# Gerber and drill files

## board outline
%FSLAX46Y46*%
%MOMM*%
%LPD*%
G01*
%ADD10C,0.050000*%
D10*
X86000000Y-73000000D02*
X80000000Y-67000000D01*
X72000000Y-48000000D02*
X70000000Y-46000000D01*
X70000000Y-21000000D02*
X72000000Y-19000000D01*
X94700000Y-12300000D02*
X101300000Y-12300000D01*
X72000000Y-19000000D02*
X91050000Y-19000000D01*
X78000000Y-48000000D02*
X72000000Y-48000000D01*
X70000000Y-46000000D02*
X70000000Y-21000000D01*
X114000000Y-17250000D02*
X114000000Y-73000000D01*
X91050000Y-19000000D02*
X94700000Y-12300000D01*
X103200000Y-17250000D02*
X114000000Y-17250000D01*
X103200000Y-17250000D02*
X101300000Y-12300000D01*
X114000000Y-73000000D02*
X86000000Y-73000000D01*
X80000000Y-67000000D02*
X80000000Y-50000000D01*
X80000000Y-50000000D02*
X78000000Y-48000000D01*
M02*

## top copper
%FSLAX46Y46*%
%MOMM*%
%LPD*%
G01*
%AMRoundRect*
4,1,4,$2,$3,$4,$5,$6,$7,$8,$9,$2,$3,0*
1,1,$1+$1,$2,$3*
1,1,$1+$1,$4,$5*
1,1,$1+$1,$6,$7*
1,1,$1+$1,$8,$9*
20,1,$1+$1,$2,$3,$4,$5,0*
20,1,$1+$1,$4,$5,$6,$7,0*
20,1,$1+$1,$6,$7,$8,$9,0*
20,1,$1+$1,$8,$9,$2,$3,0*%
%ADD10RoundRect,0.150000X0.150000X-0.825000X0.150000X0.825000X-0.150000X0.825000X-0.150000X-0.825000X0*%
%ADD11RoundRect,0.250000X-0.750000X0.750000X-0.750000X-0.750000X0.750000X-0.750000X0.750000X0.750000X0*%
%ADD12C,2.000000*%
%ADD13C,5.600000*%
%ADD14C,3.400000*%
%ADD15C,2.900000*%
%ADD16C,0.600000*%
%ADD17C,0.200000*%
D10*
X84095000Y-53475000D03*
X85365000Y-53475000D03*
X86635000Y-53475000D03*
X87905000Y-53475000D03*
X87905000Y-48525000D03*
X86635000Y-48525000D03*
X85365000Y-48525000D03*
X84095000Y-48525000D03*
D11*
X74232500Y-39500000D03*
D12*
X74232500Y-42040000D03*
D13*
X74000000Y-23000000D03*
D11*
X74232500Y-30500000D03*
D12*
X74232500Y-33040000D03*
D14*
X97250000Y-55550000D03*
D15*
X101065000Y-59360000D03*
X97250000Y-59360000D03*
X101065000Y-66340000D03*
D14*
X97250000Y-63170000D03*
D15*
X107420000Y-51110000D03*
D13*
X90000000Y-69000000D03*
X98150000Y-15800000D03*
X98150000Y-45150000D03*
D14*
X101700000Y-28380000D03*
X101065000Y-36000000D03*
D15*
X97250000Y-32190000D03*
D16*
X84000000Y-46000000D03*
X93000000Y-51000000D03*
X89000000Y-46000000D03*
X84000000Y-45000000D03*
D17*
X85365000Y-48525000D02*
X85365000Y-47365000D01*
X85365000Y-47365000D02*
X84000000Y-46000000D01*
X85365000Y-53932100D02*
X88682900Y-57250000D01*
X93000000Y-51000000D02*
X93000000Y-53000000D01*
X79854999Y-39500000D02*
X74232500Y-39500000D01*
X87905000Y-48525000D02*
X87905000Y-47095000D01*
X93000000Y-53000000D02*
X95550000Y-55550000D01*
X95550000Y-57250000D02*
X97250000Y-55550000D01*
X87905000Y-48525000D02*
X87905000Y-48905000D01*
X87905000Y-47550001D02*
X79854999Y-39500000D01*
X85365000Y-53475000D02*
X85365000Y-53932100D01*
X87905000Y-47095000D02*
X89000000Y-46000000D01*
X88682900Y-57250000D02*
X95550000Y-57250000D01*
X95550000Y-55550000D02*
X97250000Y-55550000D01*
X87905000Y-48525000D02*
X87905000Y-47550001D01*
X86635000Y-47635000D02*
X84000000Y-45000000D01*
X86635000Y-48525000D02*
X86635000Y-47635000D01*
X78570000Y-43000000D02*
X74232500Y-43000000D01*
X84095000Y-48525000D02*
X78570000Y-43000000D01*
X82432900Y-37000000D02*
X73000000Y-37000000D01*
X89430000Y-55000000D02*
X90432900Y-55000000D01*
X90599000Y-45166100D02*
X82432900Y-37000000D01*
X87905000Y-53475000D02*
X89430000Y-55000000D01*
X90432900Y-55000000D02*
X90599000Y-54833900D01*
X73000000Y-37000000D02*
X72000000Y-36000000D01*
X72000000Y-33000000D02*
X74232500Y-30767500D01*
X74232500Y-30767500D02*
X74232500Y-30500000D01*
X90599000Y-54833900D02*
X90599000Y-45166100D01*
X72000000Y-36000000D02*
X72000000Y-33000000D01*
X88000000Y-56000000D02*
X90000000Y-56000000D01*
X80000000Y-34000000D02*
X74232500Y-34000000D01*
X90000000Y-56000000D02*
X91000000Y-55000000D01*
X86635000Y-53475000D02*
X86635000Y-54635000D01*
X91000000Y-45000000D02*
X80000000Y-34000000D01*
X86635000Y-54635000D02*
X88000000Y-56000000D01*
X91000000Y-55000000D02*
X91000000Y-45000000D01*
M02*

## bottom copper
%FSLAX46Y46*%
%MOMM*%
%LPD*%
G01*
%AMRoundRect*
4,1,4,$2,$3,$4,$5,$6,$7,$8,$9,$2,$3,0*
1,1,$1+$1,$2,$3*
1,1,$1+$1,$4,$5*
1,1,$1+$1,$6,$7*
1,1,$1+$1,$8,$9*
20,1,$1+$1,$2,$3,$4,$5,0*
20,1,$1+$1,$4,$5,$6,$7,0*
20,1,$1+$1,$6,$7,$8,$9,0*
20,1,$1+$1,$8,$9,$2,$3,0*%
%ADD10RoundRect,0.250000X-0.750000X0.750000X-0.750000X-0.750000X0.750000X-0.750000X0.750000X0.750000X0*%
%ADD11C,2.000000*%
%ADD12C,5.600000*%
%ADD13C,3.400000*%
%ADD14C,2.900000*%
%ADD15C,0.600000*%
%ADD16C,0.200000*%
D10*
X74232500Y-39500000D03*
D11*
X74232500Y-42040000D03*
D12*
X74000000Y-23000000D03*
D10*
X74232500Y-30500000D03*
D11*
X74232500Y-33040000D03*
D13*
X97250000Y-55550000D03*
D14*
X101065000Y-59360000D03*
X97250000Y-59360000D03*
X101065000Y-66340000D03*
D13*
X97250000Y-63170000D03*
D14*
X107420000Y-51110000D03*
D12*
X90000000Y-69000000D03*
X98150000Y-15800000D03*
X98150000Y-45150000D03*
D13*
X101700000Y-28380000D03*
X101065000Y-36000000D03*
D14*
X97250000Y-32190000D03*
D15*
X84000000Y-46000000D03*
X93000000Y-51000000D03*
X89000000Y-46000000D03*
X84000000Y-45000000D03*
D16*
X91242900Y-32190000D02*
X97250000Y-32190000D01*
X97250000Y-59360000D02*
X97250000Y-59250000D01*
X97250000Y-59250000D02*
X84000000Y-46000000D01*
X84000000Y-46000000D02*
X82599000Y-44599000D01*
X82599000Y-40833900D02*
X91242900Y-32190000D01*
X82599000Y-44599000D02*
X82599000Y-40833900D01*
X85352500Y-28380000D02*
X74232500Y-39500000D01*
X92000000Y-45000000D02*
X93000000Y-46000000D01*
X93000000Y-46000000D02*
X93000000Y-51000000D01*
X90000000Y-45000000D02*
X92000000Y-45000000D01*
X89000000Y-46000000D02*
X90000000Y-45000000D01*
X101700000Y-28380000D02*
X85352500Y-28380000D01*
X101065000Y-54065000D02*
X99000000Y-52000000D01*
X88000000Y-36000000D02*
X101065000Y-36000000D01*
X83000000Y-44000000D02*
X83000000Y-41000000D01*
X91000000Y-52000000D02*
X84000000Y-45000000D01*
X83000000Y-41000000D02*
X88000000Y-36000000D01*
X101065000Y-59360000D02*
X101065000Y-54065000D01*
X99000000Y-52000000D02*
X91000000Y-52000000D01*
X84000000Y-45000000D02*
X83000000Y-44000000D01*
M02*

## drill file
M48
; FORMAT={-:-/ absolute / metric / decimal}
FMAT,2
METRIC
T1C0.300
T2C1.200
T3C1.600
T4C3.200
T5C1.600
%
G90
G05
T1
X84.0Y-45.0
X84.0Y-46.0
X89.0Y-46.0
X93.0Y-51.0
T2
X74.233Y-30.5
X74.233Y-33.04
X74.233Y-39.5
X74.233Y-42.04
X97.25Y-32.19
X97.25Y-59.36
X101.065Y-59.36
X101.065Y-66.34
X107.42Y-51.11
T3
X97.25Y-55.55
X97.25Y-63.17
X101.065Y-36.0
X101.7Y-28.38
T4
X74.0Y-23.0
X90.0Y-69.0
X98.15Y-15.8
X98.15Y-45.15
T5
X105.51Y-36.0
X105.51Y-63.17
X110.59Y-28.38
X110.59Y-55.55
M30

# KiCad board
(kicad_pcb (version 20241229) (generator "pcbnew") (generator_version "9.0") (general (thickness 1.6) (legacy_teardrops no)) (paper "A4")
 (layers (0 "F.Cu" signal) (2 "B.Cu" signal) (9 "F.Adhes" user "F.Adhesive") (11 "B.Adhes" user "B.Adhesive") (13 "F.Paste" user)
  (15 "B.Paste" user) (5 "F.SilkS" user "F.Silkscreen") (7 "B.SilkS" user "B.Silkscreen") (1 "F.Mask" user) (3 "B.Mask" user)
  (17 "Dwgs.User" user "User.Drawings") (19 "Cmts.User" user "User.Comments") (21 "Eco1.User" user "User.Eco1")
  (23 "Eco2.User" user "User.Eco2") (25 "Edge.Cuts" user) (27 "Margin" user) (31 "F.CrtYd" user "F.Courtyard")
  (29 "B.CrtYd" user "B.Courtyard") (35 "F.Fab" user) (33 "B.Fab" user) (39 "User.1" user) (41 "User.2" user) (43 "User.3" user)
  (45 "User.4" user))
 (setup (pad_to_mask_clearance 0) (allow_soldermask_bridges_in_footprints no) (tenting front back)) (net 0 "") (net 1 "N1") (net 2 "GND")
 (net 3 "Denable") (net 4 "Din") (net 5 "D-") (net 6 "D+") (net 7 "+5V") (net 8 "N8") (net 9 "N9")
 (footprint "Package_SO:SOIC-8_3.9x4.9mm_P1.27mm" (layer "F.Cu") (at 86 51 90)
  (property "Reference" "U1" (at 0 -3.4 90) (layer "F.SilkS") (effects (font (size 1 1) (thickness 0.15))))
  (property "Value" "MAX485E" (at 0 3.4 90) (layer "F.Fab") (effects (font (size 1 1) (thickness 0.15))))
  (pad "1" smd roundrect (at -2.475 -1.905 90) (size 1.95 0.6) (layers "F.Cu" "F.Mask" "F.Paste") (roundrect_rratio 0.25) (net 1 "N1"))
  (pad "2" smd roundrect (at -2.475 -0.635 90) (size 1.95 0.6) (layers "F.Cu" "F.Mask" "F.Paste") (roundrect_rratio 0.25) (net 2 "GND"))
  (pad "3" smd roundrect (at -2.475 0.635 90) (size 1.95 0.6) (layers "F.Cu" "F.Mask" "F.Paste") (roundrect_rratio 0.25) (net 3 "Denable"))
  (pad "4" smd roundrect (at -2.475 1.905 90) (size 1.95 0.6) (layers "F.Cu" "F.Mask" "F.Paste") (roundrect_rratio 0.25) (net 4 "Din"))
  (pad "5" smd roundrect (at 2.475 1.905 90) (size 1.95 0.6) (layers "F.Cu" "F.Mask" "F.Paste") (roundrect_rratio 0.25) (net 2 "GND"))
  (pad "6" smd roundrect (at 2.475 0.635 90) (size 1.95 0.6) (layers "F.Cu" "F.Mask" "F.Paste") (roundrect_rratio 0.25) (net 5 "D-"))
  (pad "7" smd roundrect (at 2.475 -0.635 90) (size 1.95 0.6) (layers "F.Cu" "F.Mask" "F.Paste") (roundrect_rratio 0.25) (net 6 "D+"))
  (pad "8" smd roundrect (at 2.475 -1.905 90) (size 1.95 0.6) (layers "F.Cu" "F.Mask" "F.Paste") (roundrect_rratio 0.25) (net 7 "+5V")))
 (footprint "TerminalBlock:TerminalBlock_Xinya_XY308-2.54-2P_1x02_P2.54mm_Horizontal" (layer "F.Cu") (at 74.2325 39.5 -90)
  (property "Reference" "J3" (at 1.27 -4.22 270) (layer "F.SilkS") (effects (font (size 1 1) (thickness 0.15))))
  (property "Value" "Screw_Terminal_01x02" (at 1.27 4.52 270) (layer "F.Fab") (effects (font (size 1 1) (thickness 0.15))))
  (pad "1" thru_hole roundrect (at 0 0 270) (size 2 2) (drill 1.2) (layers "*.Cu" "*.Mask") (remove_unused_layers no)
   (roundrect_rratio 0.125) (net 2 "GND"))
  (pad "2" thru_hole circle (at 2.54 0 270) (size 2 2) (drill 1.2) (layers "*.Cu" "*.Mask") (remove_unused_layers no) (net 7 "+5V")))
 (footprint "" (layer "F.Cu") (at 74 23)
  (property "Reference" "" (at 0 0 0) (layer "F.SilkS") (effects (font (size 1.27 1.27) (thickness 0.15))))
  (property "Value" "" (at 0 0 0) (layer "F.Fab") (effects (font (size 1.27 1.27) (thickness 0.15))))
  (pad "1" thru_hole circle (at 0 0) (size 5.6 5.6) (drill 3.2) (layers "*.Cu" "*.Mask") (remove_unused_layers no) (zone_connect 2)))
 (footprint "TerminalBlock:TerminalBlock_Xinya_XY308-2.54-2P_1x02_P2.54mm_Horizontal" (layer "F.Cu") (at 74.2325 30.5 -90)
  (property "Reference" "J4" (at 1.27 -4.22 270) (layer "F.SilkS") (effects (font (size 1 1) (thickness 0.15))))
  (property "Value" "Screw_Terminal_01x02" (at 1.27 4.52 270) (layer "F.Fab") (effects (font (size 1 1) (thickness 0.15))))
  (pad "1" thru_hole roundrect (at 0 0 270) (size 2 2) (drill 1.2) (layers "*.Cu" "*.Mask") (remove_unused_layers no)
   (roundrect_rratio 0.125) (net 4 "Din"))
  (pad "2" thru_hole circle (at 2.54 0 270) (size 2 2) (drill 1.2) (layers "*.Cu" "*.Mask") (remove_unused_layers no) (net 3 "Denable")))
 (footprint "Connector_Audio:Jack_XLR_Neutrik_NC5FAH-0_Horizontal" (layer "F.Cu") (at 97.25 55.55)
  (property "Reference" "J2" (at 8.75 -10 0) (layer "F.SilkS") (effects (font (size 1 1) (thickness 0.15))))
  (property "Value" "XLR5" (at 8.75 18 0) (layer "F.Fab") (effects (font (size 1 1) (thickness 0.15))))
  (pad "" np_thru_hole circle (at 8.26 7.62) (size 1.6 1.6) (drill 1.6) (layers "*.Cu" "*.Mask"))
  (pad "" np_thru_hole circle (at 13.34 0) (size 1.6 1.6) (drill 1.6) (layers "*.Cu" "*.Mask"))
  (pad "1" thru_hole circle (at 0 0) (size 3.4 3.4) (drill 1.6) (layers "*.Cu" "*.Mask") (remove_unused_layers no) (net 2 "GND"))
  (pad "2" thru_hole circle (at 3.815 3.81) (size 2.9 2.9) (drill 1.2) (layers "*.Cu" "*.Mask") (remove_unused_layers no) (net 5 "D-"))
  (pad "3" thru_hole circle (at 0 3.81) (size 2.9 2.9) (drill 1.2) (layers "*.Cu" "*.Mask") (remove_unused_layers no) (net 6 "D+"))
  (pad "4" thru_hole circle (at 3.815 10.79) (size 2.9 2.9) (drill 1.2) (layers "*.Cu" "*.Mask") (remove_unused_layers no) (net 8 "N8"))
  (pad "5" thru_hole circle (at 0 7.62) (size 3.4 3.4) (drill 1.6) (layers "*.Cu" "*.Mask") (remove_unused_layers no) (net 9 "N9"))
  (pad "G" thru_hole circle (at 10.17 -4.44) (size 2.9 2.9) (drill 1.2) (layers "*.Cu" "*.Mask") (remove_unused_layers no)))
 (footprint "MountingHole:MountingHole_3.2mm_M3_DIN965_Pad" (layer "F.Cu") (at 90 69)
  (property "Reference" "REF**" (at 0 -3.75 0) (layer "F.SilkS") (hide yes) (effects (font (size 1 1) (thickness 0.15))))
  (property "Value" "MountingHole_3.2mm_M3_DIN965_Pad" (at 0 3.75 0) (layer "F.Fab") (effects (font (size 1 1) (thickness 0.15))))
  (pad "1" thru_hole circle (at 0 0) (size 5.6 5.6) (drill 3.2) (layers "*.Cu" "*.Mask") (remove_unused_layers no) (zone_connect 2)))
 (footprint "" (layer "F.Cu") (at 98.15 15.8)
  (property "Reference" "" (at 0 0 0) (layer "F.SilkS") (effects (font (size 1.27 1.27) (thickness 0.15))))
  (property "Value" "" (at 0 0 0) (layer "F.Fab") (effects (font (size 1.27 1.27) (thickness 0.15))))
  (pad "1" thru_hole circle (at 0 0) (size 5.6 5.6) (drill 3.2) (layers "*.Cu" "*.Mask") (remove_unused_layers no) (zone_connect 2)))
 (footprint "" (layer "F.Cu") (at 98.15 45.15)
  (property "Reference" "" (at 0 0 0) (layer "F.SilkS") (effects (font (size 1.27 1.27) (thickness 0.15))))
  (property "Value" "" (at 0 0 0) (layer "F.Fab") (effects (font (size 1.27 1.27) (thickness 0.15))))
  (pad "1" thru_hole circle (at 0 0) (size 5.6 5.6) (drill 3.2) (layers "*.Cu" "*.Mask") (remove_unused_layers no) (zone_connect 2)))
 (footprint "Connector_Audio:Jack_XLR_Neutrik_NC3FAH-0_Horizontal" (layer "F.Cu") (at 101.7 28.38)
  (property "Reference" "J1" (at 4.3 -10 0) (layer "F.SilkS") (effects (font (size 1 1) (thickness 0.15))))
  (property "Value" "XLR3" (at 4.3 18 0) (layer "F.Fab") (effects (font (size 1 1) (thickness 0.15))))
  (pad "" np_thru_hole circle (at 3.81 7.62) (size 1.6 1.6) (drill 1.6) (layers "*.Cu" "*.Mask"))
  (pad "" np_thru_hole circle (at 8.89 0) (size 1.6 1.6) (drill 1.6) (layers "*.Cu" "*.Mask"))
  (pad "1" thru_hole circle (at 0 0) (size 3.4 3.4) (drill 1.6) (layers "*.Cu" "*.Mask") (remove_unused_layers no) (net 2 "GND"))
  (pad "2" thru_hole circle (at -0.635 7.62) (size 3.4 3.4) (drill 1.6) (layers "*.Cu" "*.Mask") (remove_unused_layers no) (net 5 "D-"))
  (pad "3" thru_hole circle (at -4.45 3.81) (size 2.9 2.9) (drill 1.2) (layers "*.Cu" "*.Mask") (remove_unused_layers no) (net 6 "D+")))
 (gr_line (start 86 73) (end 80 67) (stroke (width 0.05) (type default)) (layer "Edge.Cuts"))
 (gr_line (start 72 48) (end 70 46) (stroke (width 0.05) (type default)) (layer "Edge.Cuts"))
 (gr_line (start 70 21) (end 72 19) (stroke (width 0.05) (type default)) (layer "Edge.Cuts"))
 (gr_line (start 94.7 12.3) (end 101.3 12.3) (stroke (width 0.05) (type default)) (layer "Edge.Cuts"))
 (gr_line (start 72 19) (end 91.05 19) (stroke (width 0.05) (type default)) (layer "Edge.Cuts"))
 (gr_line (start 78 48) (end 72 48) (stroke (width 0.05) (type default)) (layer "Edge.Cuts"))
 (gr_line (start 70 46) (end 70 21) (stroke (width 0.05) (type default)) (layer "Edge.Cuts"))
 (gr_line (start 114 17.25) (end 114 73) (stroke (width 0.05) (type default)) (layer "Edge.Cuts"))
 (gr_line (start 91.05 19) (end 94.7 12.3) (stroke (width 0.05) (type default)) (layer "Edge.Cuts"))
 (gr_line (start 103.2 17.25) (end 114 17.25) (stroke (width 0.05) (type default)) (layer "Edge.Cuts"))
 (gr_line (start 103.2 17.25) (end 101.3 12.3) (stroke (width 0.05) (type default)) (layer "Edge.Cuts"))
 (gr_line (start 114 73) (end 86 73) (stroke (width 0.05) (type default)) (layer "Edge.Cuts"))
 (gr_line (start 80 67) (end 80 50) (stroke (width 0.05) (type default)) (layer "Edge.Cuts"))
 (gr_line (start 80 50) (end 78 48) (stroke (width 0.05) (type default)) (layer "Edge.Cuts"))
 (segment (start 85.365 48.525) (end 85.365 47.365) (width 0.2) (layer "F.Cu") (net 6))
 (segment (start 85.365 47.365) (end 84 46) (width 0.2) (layer "F.Cu") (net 6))
 (via (at 84 46) (size 0.6) (drill 0.3) (layers "F.Cu" "B.Cu") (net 6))
 (segment (start 91.2429 32.19) (end 97.25 32.19) (width 0.2) (layer "B.Cu") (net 6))
 (segment (start 97.25 59.36) (end 97.25 59.25) (width 0.2) (layer "B.Cu") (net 6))
 (segment (start 97.25 59.25) (end 84 46) (width 0.2) (layer "B.Cu") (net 6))
 (segment (start 84 46) (end 82.599 44.599) (width 0.2) (layer "B.Cu") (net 6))
 (segment (start 82.599 40.8339) (end 91.2429 32.19) (width 0.2) (layer "B.Cu") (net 6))
 (segment (start 82.599 44.599) (end 82.599 40.8339) (width 0.2) (layer "B.Cu") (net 6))
 (segment (start 85.365 53.9321) (end 88.6829 57.25) (width 0.2) (layer "F.Cu") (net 2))
 (segment (start 93 51) (end 93 53) (width 0.2) (layer "F.Cu") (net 2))
 (segment (start 79.854999 39.5) (end 74.2325 39.5) (width 0.2) (layer "F.Cu") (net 2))
 (segment (start 87.905 48.525) (end 87.905 47.095) (width 0.2) (layer "F.Cu") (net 2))
 (segment (start 93 53) (end 95.55 55.55) (width 0.2) (layer "F.Cu") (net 2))
 (segment (start 95.55 57.25) (end 97.25 55.55) (width 0.2) (layer "F.Cu") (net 2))
 (segment (start 87.905 48.525) (end 87.905 48.905) (width 0.2) (layer "F.Cu") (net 2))
 (segment (start 87.905 47.550001) (end 79.854999 39.5) (width 0.2) (layer "F.Cu") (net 2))
 (segment (start 85.365 53.475) (end 85.365 53.9321) (width 0.2) (layer "F.Cu") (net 2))
 (segment (start 87.905 47.095) (end 89 46) (width 0.2) (layer "F.Cu") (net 2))
 (segment (start 88.6829 57.25) (end 95.55 57.25) (width 0.2) (layer "F.Cu") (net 2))
 (segment (start 95.55 55.55) (end 97.25 55.55) (width 0.2) (layer "F.Cu") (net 2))
 (segment (start 87.905 48.525) (end 87.905 47.550001) (width 0.2) (layer "F.Cu") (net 2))
 (via (at 93 51) (size 0.6) (drill 0.3) (layers "F.Cu" "B.Cu") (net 2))
 (via (at 89 46) (size 0.6) (drill 0.3) (layers "F.Cu" "B.Cu") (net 2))
 (segment (start 85.3525 28.38) (end 74.2325 39.5) (width 0.2) (layer "B.Cu") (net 2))
 (segment (start 92 45) (end 93 46) (width 0.2) (layer "B.Cu") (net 2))
 (segment (start 93 46) (end 93 51) (width 0.2) (layer "B.Cu") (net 2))
 (segment (start 90 45) (end 92 45) (width 0.2) (layer "B.Cu") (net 2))
 (segment (start 89 46) (end 90 45) (width 0.2) (layer "B.Cu") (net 2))
 (segment (start 101.7 28.38) (end 85.3525 28.38) (width 0.2) (layer "B.Cu") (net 2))
 (segment (start 86.635 47.635) (end 84 45) (width 0.2) (layer "F.Cu") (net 5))
 (segment (start 86.635 48.525) (end 86.635 47.635) (width 0.2) (layer "F.Cu") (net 5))
 (via (at 84 45) (size 0.6) (drill 0.3) (layers "F.Cu" "B.Cu") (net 5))
 (segment (start 101.065 54.065) (end 99 52) (width 0.2) (layer "B.Cu") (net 5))
 (segment (start 88 36) (end 101.065 36) (width 0.2) (layer "B.Cu") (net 5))
 (segment (start 83 44) (end 83 41) (width 0.2) (layer "B.Cu") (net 5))
 (segment (start 91 52) (end 84 45) (width 0.2) (layer "B.Cu") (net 5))
 (segment (start 83 41) (end 88 36) (width 0.2) (layer "B.Cu") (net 5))
 (segment (start 101.065 59.36) (end 101.065 54.065) (width 0.2) (layer "B.Cu") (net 5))
 (segment (start 99 52) (end 91 52) (width 0.2) (layer "B.Cu") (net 5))
 (segment (start 84 45) (end 83 44) (width 0.2) (layer "B.Cu") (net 5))
 (segment (start 78.57 43) (end 74.2325 43) (width 0.2) (layer "F.Cu") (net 7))
 (segment (start 84.095 48.525) (end 78.57 43) (width 0.2) (layer "F.Cu") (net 7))
 (segment (start 82.4329 37) (end 73 37) (width 0.2) (layer "F.Cu") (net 4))
 (segment (start 89.43 55) (end 90.4329 55) (width 0.2) (layer "F.Cu") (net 4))
 (segment (start 90.599 45.1661) (end 82.4329 37) (width 0.2) (layer "F.Cu") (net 4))
 (segment (start 87.905 53.475) (end 89.43 55) (width 0.2) (layer "F.Cu") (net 4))
 (segment (start 90.4329 55) (end 90.599 54.8339) (width 0.2) (layer "F.Cu") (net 4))
 (segment (start 73 37) (end 72 36) (width 0.2) (layer "F.Cu") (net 4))
 (segment (start 72 33) (end 74.2325 30.7675) (width 0.2) (layer "F.Cu") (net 4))
 (segment (start 74.2325 30.7675) (end 74.2325 30.5) (width 0.2) (layer "F.Cu") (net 4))
 (segment (start 90.599 54.8339) (end 90.599 45.1661) (width 0.2) (layer "F.Cu") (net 4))
 (segment (start 72 36) (end 72 33) (width 0.2) (layer "F.Cu") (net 4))
 (segment (start 88 56) (end 90 56) (width 0.2) (layer "F.Cu") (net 3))
 (segment (start 80 34) (end 74.2325 34) (width 0.2) (layer "F.Cu") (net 3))
 (segment (start 90 56) (end 91 55) (width 0.2) (layer "F.Cu") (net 3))
 (segment (start 86.635 53.475) (end 86.635 54.635) (width 0.2) (layer "F.Cu") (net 3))
 (segment (start 91 45) (end 80 34) (width 0.2) (layer "F.Cu") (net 3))
 (segment (start 86.635 54.635) (end 88 56) (width 0.2) (layer "F.Cu") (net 3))
 (segment (start 91 55) (end 91 45) (width 0.2) (layer "F.Cu") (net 3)))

